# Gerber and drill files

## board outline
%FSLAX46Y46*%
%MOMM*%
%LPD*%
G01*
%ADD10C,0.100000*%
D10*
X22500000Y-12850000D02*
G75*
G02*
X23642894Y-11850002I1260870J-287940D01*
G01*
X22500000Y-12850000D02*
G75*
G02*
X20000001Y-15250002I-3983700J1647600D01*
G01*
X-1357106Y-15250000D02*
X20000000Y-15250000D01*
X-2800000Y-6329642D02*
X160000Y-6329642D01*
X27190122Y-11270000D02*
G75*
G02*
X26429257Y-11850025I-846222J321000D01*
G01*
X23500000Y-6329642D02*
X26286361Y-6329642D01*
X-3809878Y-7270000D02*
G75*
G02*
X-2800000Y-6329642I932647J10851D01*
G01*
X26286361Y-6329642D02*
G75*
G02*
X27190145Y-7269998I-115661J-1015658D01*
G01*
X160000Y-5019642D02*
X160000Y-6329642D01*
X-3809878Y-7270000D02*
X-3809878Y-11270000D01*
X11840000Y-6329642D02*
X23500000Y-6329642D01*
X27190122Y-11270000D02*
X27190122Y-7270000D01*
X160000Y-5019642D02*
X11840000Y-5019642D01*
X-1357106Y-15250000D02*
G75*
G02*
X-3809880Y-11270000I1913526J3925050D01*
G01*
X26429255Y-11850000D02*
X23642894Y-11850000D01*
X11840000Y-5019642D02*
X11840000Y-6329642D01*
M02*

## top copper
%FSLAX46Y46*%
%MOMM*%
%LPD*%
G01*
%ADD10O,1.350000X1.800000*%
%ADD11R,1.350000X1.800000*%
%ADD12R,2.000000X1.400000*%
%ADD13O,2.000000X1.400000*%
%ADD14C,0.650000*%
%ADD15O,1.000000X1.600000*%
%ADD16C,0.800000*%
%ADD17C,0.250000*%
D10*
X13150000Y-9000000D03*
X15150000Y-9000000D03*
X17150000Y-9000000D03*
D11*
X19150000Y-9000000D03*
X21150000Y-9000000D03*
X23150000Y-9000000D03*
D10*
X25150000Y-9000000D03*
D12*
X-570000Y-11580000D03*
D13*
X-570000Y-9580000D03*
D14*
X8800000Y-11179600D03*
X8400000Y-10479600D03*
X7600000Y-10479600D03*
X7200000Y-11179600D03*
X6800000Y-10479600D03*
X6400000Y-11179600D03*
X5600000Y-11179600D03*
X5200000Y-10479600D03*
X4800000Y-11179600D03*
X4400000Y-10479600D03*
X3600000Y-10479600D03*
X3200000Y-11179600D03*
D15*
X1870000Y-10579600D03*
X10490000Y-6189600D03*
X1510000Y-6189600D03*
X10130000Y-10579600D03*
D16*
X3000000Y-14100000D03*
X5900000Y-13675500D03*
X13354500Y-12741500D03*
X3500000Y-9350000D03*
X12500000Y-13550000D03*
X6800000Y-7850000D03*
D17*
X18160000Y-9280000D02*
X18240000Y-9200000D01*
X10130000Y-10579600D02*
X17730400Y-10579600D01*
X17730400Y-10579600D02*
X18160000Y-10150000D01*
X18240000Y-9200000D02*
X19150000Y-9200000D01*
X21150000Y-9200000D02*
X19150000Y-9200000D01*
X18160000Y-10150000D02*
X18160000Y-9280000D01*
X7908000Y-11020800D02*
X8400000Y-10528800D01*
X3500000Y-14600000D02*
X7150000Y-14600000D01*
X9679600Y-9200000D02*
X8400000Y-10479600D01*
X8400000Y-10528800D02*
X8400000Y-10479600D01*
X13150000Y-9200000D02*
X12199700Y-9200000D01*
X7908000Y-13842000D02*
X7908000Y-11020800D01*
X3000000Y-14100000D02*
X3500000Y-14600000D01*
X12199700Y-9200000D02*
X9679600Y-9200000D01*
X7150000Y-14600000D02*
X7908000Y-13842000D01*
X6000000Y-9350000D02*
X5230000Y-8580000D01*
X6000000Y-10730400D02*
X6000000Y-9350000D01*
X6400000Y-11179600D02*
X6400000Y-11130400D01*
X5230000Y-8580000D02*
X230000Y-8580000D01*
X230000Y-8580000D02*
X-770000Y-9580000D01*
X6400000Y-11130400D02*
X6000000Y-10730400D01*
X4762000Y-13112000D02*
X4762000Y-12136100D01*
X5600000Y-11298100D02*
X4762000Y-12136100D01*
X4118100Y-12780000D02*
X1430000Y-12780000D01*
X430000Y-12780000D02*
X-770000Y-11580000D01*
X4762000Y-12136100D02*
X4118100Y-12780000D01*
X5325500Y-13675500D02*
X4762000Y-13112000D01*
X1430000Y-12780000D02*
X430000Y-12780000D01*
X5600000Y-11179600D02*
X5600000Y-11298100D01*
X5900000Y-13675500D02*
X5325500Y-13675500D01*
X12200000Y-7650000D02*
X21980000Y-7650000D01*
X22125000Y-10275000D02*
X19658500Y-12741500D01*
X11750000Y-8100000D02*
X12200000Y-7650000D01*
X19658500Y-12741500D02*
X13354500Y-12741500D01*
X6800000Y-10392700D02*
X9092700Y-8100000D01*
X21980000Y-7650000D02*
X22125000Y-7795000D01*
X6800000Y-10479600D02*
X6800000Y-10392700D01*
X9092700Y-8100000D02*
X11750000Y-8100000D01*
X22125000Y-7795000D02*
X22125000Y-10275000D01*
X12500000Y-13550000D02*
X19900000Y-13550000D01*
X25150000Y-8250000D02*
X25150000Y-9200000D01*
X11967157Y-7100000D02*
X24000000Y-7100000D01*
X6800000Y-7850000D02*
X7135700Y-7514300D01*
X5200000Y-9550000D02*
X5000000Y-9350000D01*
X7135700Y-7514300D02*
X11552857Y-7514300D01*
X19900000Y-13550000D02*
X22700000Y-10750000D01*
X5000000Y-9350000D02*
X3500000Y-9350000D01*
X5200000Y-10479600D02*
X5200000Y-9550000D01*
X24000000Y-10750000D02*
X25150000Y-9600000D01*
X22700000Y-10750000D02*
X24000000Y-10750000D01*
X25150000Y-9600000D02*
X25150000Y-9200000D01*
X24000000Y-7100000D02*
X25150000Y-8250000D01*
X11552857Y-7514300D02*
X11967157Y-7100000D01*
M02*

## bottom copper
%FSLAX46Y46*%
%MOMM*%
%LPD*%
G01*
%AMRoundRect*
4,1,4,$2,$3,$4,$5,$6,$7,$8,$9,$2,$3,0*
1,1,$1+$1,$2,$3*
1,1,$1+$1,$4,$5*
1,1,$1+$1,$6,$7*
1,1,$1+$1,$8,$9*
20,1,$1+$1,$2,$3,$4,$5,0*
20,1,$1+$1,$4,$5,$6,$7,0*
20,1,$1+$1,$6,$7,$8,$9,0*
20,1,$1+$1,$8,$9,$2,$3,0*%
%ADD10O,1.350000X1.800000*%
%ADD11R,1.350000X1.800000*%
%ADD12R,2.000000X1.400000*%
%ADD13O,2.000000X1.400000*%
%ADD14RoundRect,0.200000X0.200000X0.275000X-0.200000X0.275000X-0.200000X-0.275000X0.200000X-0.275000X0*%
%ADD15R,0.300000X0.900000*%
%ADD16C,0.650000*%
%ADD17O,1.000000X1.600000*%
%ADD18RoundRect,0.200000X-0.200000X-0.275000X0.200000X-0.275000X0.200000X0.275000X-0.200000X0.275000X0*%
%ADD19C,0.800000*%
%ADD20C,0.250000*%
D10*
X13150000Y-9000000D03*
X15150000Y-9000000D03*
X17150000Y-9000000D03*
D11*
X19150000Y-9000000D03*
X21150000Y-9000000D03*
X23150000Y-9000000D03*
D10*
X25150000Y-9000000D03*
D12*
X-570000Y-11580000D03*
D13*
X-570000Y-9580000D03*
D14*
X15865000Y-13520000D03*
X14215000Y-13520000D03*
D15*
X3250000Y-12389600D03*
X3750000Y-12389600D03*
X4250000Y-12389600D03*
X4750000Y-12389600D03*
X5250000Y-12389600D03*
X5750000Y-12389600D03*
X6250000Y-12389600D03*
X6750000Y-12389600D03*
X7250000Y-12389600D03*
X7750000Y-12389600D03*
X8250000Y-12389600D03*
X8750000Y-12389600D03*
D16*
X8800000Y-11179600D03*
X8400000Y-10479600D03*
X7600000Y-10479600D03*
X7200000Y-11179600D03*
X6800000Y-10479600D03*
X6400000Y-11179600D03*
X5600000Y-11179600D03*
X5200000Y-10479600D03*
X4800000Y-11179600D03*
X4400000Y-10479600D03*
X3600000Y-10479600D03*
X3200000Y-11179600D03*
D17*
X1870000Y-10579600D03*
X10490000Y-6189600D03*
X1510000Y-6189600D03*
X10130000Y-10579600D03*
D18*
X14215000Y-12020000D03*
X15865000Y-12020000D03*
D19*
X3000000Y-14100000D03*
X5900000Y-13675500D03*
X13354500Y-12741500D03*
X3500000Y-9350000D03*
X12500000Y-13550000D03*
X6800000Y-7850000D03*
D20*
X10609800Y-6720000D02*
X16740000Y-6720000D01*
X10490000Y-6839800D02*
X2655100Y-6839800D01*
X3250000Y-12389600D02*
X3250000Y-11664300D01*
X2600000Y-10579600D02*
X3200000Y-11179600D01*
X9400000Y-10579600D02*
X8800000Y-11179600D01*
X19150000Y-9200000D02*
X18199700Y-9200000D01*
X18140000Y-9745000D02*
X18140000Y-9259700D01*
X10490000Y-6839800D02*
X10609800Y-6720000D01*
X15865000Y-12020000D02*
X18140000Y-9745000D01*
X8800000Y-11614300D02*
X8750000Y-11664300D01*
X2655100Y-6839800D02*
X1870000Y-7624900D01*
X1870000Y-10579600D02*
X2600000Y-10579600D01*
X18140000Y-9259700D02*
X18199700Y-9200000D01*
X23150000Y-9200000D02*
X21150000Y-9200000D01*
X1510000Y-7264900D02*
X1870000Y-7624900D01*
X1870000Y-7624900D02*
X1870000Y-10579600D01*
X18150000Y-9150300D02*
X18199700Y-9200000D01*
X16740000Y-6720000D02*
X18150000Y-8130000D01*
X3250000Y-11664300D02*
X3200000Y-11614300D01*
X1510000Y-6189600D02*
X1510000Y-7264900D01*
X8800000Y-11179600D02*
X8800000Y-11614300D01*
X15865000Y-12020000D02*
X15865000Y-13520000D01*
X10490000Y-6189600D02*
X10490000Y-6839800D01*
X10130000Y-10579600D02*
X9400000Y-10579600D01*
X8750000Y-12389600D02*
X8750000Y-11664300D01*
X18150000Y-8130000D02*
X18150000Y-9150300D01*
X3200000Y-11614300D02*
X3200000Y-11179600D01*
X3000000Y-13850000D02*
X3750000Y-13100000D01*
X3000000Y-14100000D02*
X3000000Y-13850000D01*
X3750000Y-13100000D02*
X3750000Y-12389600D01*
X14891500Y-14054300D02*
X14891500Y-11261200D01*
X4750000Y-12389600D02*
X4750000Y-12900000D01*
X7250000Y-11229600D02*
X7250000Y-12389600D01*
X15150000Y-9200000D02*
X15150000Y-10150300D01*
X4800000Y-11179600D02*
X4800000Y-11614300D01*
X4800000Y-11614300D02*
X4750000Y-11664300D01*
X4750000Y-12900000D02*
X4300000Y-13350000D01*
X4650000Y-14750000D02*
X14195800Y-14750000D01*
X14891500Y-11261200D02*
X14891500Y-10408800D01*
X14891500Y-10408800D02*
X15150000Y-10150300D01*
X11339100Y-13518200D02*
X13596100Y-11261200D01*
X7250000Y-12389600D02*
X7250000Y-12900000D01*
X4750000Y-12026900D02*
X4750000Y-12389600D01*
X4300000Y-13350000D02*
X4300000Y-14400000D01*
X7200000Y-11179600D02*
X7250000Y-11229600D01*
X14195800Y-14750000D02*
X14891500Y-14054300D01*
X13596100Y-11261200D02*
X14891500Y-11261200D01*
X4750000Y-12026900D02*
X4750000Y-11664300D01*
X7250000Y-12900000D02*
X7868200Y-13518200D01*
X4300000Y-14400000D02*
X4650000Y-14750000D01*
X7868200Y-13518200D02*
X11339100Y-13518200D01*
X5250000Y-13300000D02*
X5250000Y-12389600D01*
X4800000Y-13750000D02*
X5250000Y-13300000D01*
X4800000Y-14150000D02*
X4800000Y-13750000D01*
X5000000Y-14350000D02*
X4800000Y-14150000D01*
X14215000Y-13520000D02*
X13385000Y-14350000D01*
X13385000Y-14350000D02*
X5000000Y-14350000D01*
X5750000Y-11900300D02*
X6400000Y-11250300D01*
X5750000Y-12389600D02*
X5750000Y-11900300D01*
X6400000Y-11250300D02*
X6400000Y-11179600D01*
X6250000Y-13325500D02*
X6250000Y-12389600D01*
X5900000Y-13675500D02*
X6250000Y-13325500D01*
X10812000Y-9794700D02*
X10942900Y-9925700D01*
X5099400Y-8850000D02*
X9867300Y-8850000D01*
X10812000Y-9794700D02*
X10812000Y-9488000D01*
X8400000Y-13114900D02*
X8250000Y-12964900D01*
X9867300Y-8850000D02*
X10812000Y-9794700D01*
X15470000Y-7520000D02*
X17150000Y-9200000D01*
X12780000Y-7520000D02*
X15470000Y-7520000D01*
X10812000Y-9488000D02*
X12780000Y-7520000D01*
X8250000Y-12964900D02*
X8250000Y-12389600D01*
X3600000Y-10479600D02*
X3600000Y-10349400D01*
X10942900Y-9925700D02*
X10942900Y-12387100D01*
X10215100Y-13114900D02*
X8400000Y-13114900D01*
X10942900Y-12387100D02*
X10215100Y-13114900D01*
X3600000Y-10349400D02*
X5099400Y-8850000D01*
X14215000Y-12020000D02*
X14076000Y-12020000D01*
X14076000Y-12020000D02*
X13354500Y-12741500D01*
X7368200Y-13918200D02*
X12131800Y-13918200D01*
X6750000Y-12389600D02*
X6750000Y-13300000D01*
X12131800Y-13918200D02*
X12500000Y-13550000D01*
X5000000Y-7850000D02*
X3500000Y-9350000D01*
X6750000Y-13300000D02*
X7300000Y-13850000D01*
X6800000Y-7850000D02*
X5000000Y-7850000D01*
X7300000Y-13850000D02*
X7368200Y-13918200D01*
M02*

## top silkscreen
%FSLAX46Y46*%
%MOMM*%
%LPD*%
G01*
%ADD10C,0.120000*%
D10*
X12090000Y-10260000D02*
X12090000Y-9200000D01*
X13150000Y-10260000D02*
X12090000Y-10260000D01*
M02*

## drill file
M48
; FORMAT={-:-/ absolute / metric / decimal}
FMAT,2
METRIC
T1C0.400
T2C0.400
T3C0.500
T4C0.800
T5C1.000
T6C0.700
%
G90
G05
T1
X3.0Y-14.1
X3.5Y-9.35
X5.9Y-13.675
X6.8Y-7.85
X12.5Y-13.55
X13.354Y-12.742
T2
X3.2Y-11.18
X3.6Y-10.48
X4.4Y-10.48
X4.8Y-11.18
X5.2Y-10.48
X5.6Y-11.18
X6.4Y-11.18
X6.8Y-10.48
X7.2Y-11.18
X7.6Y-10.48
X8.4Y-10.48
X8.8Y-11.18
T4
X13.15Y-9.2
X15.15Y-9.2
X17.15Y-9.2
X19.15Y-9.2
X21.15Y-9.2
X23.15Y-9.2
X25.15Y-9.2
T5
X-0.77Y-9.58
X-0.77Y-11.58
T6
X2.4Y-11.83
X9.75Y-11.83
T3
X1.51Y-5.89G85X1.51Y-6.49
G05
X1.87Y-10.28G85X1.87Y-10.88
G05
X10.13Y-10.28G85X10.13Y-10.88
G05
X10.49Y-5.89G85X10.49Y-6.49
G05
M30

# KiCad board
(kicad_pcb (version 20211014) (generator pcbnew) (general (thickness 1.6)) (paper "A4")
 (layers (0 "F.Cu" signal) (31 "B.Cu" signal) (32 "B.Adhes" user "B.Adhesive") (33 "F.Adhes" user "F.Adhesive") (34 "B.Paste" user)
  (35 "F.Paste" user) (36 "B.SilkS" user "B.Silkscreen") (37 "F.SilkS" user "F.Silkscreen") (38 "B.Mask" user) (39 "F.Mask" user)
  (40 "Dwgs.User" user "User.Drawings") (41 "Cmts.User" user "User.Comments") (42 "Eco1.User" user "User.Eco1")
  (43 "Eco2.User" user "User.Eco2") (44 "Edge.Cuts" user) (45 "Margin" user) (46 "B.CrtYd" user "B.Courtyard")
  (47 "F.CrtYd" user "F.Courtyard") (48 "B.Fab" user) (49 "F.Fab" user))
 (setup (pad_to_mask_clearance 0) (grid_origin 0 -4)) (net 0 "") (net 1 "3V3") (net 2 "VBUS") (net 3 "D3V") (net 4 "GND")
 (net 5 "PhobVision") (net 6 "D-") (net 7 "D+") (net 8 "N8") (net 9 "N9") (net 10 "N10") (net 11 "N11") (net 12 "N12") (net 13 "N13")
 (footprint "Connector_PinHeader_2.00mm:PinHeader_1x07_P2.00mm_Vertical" (layer "F.Cu") (at 13.15 9.2 90)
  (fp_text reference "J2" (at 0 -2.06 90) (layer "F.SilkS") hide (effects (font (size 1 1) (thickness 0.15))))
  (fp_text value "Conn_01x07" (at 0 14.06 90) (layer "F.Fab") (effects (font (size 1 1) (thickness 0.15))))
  (fp_line (start -1.06 -1.06) (end 0 -1.06) (layer "F.SilkS") (width 0.12))
  (fp_line (start -1.06 0) (end -1.06 -1.06) (layer "F.SilkS") (width 0.12))
  (pad "1" thru_hole oval (at 0 0 90) (size 1.8 1.35) (drill 0.8 (offset 0.2 0)) (layers F&B.Cu *.Mask) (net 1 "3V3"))
  (pad "2" thru_hole oval (at 0 2 90) (size 1.8 1.35) (drill 0.8 (offset 0.2 0)) (layers F&B.Cu *.Mask) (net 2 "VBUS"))
  (pad "3" thru_hole oval (at 0 4 90) (size 1.8 1.35) (drill 0.8 (offset 0.2 0)) (layers F&B.Cu *.Mask) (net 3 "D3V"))
  (pad "4" thru_hole rect (at 0 6 90) (size 1.8 1.35) (drill 0.8 (offset 0.2 0)) (layers F&B.Cu *.Mask) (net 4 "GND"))
  (pad "5" thru_hole rect (at 0 8 90) (size 1.8 1.35) (drill 0.8 (offset 0.2 0)) (layers F&B.Cu *.Mask) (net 4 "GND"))
  (pad "6" thru_hole rect (at 0 10 90) (size 1.8 1.35) (drill 0.8 (offset 0.2 0)) (layers F&B.Cu *.Mask) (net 4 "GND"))
  (pad "7" thru_hole oval (at 0 12 90) (size 1.8 1.35) (drill 0.8 (offset 0.2 0)) (layers F&B.Cu *.Mask) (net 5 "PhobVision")))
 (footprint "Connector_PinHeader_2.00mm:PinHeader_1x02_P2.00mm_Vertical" (layer "B.Cu") (at -0.77 11.58)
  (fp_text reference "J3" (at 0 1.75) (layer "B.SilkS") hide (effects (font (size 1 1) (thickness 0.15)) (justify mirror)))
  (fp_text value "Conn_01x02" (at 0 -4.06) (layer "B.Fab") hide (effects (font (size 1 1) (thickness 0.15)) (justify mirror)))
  (pad "1" thru_hole rect locked (at 0 0) (size 2 1.4) (drill 1 (offset 0.2 0)) (layers F&B.Cu *.Mask) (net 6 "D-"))
  (pad "2" thru_hole oval locked (at 0 -2) (size 2 1.4) (drill 1 (offset 0.2 0)) (layers F&B.Cu *.Mask) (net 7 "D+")))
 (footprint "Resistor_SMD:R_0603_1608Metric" (layer "B.Cu") (at 15.04 13.52 180)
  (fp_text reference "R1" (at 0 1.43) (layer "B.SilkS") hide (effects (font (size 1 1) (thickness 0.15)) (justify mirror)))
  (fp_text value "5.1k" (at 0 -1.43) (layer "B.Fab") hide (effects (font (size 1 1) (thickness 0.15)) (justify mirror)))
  (pad "1" smd roundrect locked (at -0.825 0 180) (size 0.8 0.95) (layers "B.Cu" "B.Paste" "B.Mask") (roundrect_rratio 0.25) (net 4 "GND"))
  (pad "2" smd roundrect locked (at 0.825 0 180) (size 0.8 0.95) (layers "B.Cu" "B.Paste" "B.Mask") (roundrect_rratio 0.25) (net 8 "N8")))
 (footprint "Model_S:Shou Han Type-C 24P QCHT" (layer "B.Cu") (at 6 4.3296)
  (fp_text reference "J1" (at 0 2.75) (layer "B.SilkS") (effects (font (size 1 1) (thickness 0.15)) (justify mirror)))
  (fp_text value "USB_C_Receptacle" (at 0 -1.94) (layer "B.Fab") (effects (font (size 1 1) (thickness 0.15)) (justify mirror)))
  (pad "" np_thru_hole circle (at -3.6 7.5) (size 0.7 0.7) (drill 0.7) (layers F&B.Cu *.Mask))
  (pad "" np_thru_hole circle (at 3.75 7.5) (size 0.7 0.7) (drill 0.7) (layers F&B.Cu *.Mask))
  (pad "A1" smd rect (at -2.75 8.06) (size 0.3 0.9) (layers "B.Cu" "B.Paste" "B.Mask") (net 4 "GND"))
  (pad "A2" smd rect (at -2.25 8.06) (size 0.3 0.9) (layers "B.Cu" "B.Paste" "B.Mask") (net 1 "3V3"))
  (pad "A3" smd rect (at -1.75 8.06) (size 0.3 0.9) (layers "B.Cu" "B.Paste" "B.Mask") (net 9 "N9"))
  (pad "A4" smd rect (at -1.25 8.06) (size 0.3 0.9) (layers "B.Cu" "B.Paste" "B.Mask") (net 2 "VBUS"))
  (pad "A5" smd rect (at -0.75 8.06) (size 0.3 0.9) (layers "B.Cu" "B.Paste" "B.Mask") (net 8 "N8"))
  (pad "A6" smd rect (at -0.25 8.06) (size 0.3 0.9) (layers "B.Cu" "B.Paste" "B.Mask") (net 7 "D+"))
  (pad "A7" smd rect (at 0.25 8.06) (size 0.3 0.9) (layers "B.Cu" "B.Paste" "B.Mask") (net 6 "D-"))
  (pad "A8" smd rect (at 0.75 8.06) (size 0.3 0.9) (layers "B.Cu" "B.Paste" "B.Mask") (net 5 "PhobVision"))
  (pad "A9" smd rect (at 1.25 8.06) (size 0.3 0.9) (layers "B.Cu" "B.Paste" "B.Mask") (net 2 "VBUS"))
  (pad "A10" smd rect (at 1.75 8.06) (size 0.3 0.9) (layers "B.Cu" "B.Paste" "B.Mask") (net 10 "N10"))
  (pad "A11" smd rect (at 2.25 8.06) (size 0.3 0.9) (layers "B.Cu" "B.Paste" "B.Mask") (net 3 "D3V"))
  (pad "A12" smd rect (at 2.75 8.06) (size 0.3 0.9) (layers "B.Cu" "B.Paste" "B.Mask") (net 4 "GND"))
  (pad "B1" thru_hole circle (at 2.8 6.85) (size 0.65 0.65) (drill 0.4) (layers F&B.Cu *.Mask) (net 4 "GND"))
  (pad "B2" thru_hole circle (at 2.4 6.15) (size 0.65 0.65) (drill 0.4) (layers F&B.Cu *.Mask) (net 1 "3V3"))
  (pad "B3" thru_hole circle (at 1.6 6.15) (size 0.65 0.65) (drill 0.4) (layers F&B.Cu *.Mask) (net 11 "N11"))
  (pad "B4" thru_hole circle (at 1.2 6.85) (size 0.65 0.65) (drill 0.4) (layers F&B.Cu *.Mask) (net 2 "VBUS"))
  (pad "B5" thru_hole circle (at 0.8 6.15) (size 0.65 0.65) (drill 0.4) (layers F&B.Cu *.Mask) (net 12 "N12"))
  (pad "B6" thru_hole circle (at 0.4 6.85) (size 0.65 0.65) (drill 0.4) (layers F&B.Cu *.Mask) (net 7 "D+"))
  (pad "B7" thru_hole circle (at -0.4 6.85) (size 0.65 0.65) (drill 0.4) (layers F&B.Cu *.Mask) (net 6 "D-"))
  (pad "B8" thru_hole circle (at -0.8 6.15) (size 0.65 0.65) (drill 0.4) (layers F&B.Cu *.Mask) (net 5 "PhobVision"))
  (pad "B9" thru_hole circle (at -1.2 6.85) (size 0.65 0.65) (drill 0.4) (layers F&B.Cu *.Mask) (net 2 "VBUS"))
  (pad "B10" thru_hole circle (at -1.6 6.15) (size 0.65 0.65) (drill 0.4) (layers F&B.Cu *.Mask) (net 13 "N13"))
  (pad "B11" thru_hole circle (at -2.4 6.15) (size 0.65 0.65) (drill 0.4) (layers F&B.Cu *.Mask) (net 3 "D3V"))
  (pad "B12" thru_hole circle (at -2.8 6.85) (size 0.65 0.65) (drill 0.4) (layers F&B.Cu *.Mask) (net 4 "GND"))
  (pad "S1" thru_hole oval (at -4.13 6.25) (size 1 1.6) (drill oval 0.5 1.1) (layers F&B.Cu *.Mask) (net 4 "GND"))
  (pad "S1" thru_hole oval (at 4.49 1.86) (size 1 1.6) (drill oval 0.5 1.1) (layers F&B.Cu *.Mask) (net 4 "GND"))
  (pad "S1" thru_hole oval (at -4.49 1.86) (size 1 1.6) (drill oval 0.5 1.1) (layers F&B.Cu *.Mask) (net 4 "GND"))
  (pad "S1" thru_hole oval (at 4.13 6.25) (size 1 1.6) (drill oval 0.5 1.1) (layers F&B.Cu *.Mask) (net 4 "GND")))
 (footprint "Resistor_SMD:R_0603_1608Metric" (layer "B.Cu") (at 15.04 12.02)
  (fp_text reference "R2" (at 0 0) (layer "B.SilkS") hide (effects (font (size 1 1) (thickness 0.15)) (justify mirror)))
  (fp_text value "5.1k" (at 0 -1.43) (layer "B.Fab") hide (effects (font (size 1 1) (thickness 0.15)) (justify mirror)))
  (pad "1" smd roundrect locked (at -0.825 0) (size 0.8 0.95) (layers "B.Cu" "B.Paste" "B.Mask") (roundrect_rratio 0.25) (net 12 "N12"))
  (pad "2" smd roundrect locked (at 0.825 0) (size 0.8 0.95) (layers "B.Cu" "B.Paste" "B.Mask") (roundrect_rratio 0.25) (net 4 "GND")))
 (gr_arc (start 22.5 12.85) (mid 22.909223 12.164595) (end 23.642894 11.85) (layer "Edge.Cuts") (width 0.1))
 (gr_arc (start 22.5 12.85) (mid 21.501783 14.312274) (end 20 15.25) (layer "Edge.Cuts") (width 0.1))
 (gr_line (start -1.357106 15.25) (end 20 15.25) (layer "Edge.Cuts") (width 0.1))
 (gr_line (start -2.8 6.329642) (end 0.16 6.329642) (layer "Edge.Cuts") (width 0.1))
 (gr_arc (start 27.190122 11.27) (mid 26.892588 11.668751) (end 26.429255 11.85) (layer "Edge.Cuts") (width 0.1))
 (gr_line (start 23.5 6.329642) (end 26.286361 6.329642) (layer "Edge.Cuts") (width 0.1))
 (gr_arc (start -3.809878 7.27) (mid -3.512843 6.576547) (end -2.8 6.329642) (layer "Edge.Cuts") (width 0.1))
 (gr_arc (start 26.286361 6.329642) (mid 26.907696 6.636961) (end 27.190122 7.27) (layer "Edge.Cuts") (width 0.1))
 (gr_line (start 0.16 5.019642) (end 0.16 6.329642) (layer "Edge.Cuts") (width 0.1))
 (gr_line (start -3.809878 7.27) (end -3.809878 11.27) (layer "Edge.Cuts") (width 0.1))
 (gr_line (start 11.84 6.329642) (end 23.5 6.329642) (layer "Edge.Cuts") (width 0.1))
 (gr_line (start 27.190122 11.27) (end 27.190122 7.27) (layer "Edge.Cuts") (width 0.1))
 (gr_line (start 0.16 5.019642) (end 11.84 5.019642) (layer "Edge.Cuts") (width 0.1))
 (gr_arc (start -1.357106 15.25) (mid -3.160991 13.615898) (end -3.809878 11.27) (layer "Edge.Cuts") (width 0.1))
 (gr_line (start 26.429255 11.85) (end 23.642894 11.85) (layer "Edge.Cuts") (width 0.1))
 (gr_line (start 11.84 5.019642) (end 11.84 6.329642) (layer "Edge.Cuts") (width 0.1))
 (segment (start 18.16 9.28) (end 18.24 9.2) (width 0.25) (layer "F.Cu") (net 4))
 (segment (start 10.13 10.5796) (end 17.7304 10.5796) (width 0.25) (layer "F.Cu") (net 4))
 (segment (start 17.7304 10.5796) (end 18.16 10.15) (width 0.25) (layer "F.Cu") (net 4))
 (segment (start 18.24 9.2) (end 19.15 9.2) (width 0.25) (layer "F.Cu") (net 4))
 (segment (start 21.15 9.2) (end 19.15 9.2) (width 0.25) (layer "F.Cu") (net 4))
 (segment (start 18.16 10.15) (end 18.16 9.28) (width 0.25) (layer "F.Cu") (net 4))
 (segment (start 10.6098 6.72) (end 16.74 6.72) (width 0.25) (layer "B.Cu") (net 4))
 (segment (start 10.49 6.8398) (end 2.6551 6.8398) (width 0.25) (layer "B.Cu") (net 4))
 (segment (start 3.25 12.3896) (end 3.25 11.6643) (width 0.25) (layer "B.Cu") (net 4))
 (segment (start 2.6 10.5796) (end 3.2 11.1796) (width 0.25) (layer "B.Cu") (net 4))
 (segment (start 9.4 10.5796) (end 8.8 11.1796) (width 0.25) (layer "B.Cu") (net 4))
 (segment (start 19.15 9.2) (end 18.1997 9.2) (width 0.25) (layer "B.Cu") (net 4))
 (segment (start 18.14 9.745) (end 18.14 9.2597) (width 0.25) (layer "B.Cu") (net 4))
 (segment (start 10.49 6.8398) (end 10.6098 6.72) (width 0.25) (layer "B.Cu") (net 4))
 (segment (start 15.865 12.02) (end 18.14 9.745) (width 0.25) (layer "B.Cu") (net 4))
 (segment (start 8.8 11.6143) (end 8.75 11.6643) (width 0.25) (layer "B.Cu") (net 4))
 (segment (start 2.6551 6.8398) (end 1.87 7.6249) (width 0.25) (layer "B.Cu") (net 4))
 (segment (start 1.87 10.5796) (end 2.6 10.5796) (width 0.25) (layer "B.Cu") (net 4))
 (segment (start 18.14 9.2597) (end 18.1997 9.2) (width 0.25) (layer "B.Cu") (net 4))
 (segment (start 23.15 9.2) (end 21.15 9.2) (width 0.25) (layer "B.Cu") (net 4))
 (segment (start 1.51 7.2649) (end 1.87 7.6249) (width 0.25) (layer "B.Cu") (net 4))
 (segment (start 1.87 7.6249) (end 1.87 10.5796) (width 0.25) (layer "B.Cu") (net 4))
 (segment (start 18.15 9.1503) (end 18.1997 9.2) (width 0.25) (layer "B.Cu") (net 4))
 (segment (start 16.74 6.72) (end 18.15 8.13) (width 0.25) (layer "B.Cu") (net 4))
 (segment (start 3.25 11.6643) (end 3.2 11.6143) (width 0.25) (layer "B.Cu") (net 4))
 (segment (start 1.51 6.1896) (end 1.51 7.2649) (width 0.25) (layer "B.Cu") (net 4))
 (segment (start 8.8 11.1796) (end 8.8 11.6143) (width 0.25) (layer "B.Cu") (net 4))
 (segment (start 15.865 12.02) (end 15.865 13.52) (width 0.25) (layer "B.Cu") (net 4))
 (segment (start 10.49 6.1896) (end 10.49 6.8398) (width 0.25) (layer "B.Cu") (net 4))
 (segment (start 10.13 10.5796) (end 9.4 10.5796) (width 0.25) (layer "B.Cu") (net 4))
 (segment (start 8.75 12.3896) (end 8.75 11.6643) (width 0.25) (layer "B.Cu") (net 4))
 (segment (start 18.15 8.13) (end 18.15 9.1503) (width 0.25) (layer "B.Cu") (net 4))
 (segment (start 3.2 11.6143) (end 3.2 11.1796) (width 0.25) (layer "B.Cu") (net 4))
 (segment (start 7.908 11.0208) (end 8.4 10.5288) (width 0.25) (layer "F.Cu") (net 1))
 (segment (start 3.5 14.6) (end 7.15 14.6) (width 0.25) (layer "F.Cu") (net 1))
 (segment (start 9.6796 9.2) (end 8.4 10.4796) (width 0.25) (layer "F.Cu") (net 1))
 (segment (start 8.4 10.5288) (end 8.4 10.4796) (width 0.25) (layer "F.Cu") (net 1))
 (segment (start 13.15 9.2) (end 12.1997 9.2) (width 0.25) (layer "F.Cu") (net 1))
 (segment (start 7.908 13.842) (end 7.908 11.0208) (width 0.25) (layer "F.Cu") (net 1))
 (segment (start 3 14.1) (end 3.5 14.6) (width 0.25) (layer "F.Cu") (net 1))
 (segment (start 12.1997 9.2) (end 9.6796 9.2) (width 0.25) (layer "F.Cu") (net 1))
 (segment (start 7.15 14.6) (end 7.908 13.842) (width 0.25) (layer "F.Cu") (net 1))
 (via (at 3 14.1) (size 0.8) (drill 0.4) (layers "F.Cu" "B.Cu") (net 1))
 (segment (start 3 13.85) (end 3.75 13.1) (width 0.25) (layer "B.Cu") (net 1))
 (segment (start 3 14.1) (end 3 13.85) (width 0.25) (layer "B.Cu") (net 1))
 (segment (start 3.75 13.1) (end 3.75 12.3896) (width 0.25) (layer "B.Cu") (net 1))
 (segment (start 14.8915 14.0543) (end 14.8915 11.2612) (width 0.25) (layer "B.Cu") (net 2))
 (segment (start 4.75 12.3896) (end 4.75 12.9) (width 0.25) (layer "B.Cu") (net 2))
 (segment (start 7.25 11.2296) (end 7.25 12.3896) (width 0.25) (layer "B.Cu") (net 2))
 (segment (start 15.15 9.2) (end 15.15 10.1503) (width 0.25) (layer "B.Cu") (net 2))
 (segment (start 4.8 11.1796) (end 4.8 11.6143) (width 0.25) (layer "B.Cu") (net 2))
 (segment (start 4.8 11.6143) (end 4.75 11.6643) (width 0.25) (layer "B.Cu") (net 2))
 (segment (start 4.75 12.9) (end 4.3 13.35) (width 0.25) (layer "B.Cu") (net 2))
 (segment (start 4.65 14.75) (end 14.1958 14.75) (width 0.25) (layer "B.Cu") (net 2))
 (segment (start 14.8915 11.2612) (end 14.8915 10.4088) (width 0.25) (layer "B.Cu") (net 2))
 (segment (start 14.8915 10.4088) (end 15.15 10.1503) (width 0.25) (layer "B.Cu") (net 2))
 (segment (start 11.3391 13.5182) (end 13.5961 11.2612) (width 0.25) (layer "B.Cu") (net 2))
 (segment (start 7.25 12.3896) (end 7.25 12.9) (width 0.25) (layer "B.Cu") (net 2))
 (segment (start 4.75 12.0269) (end 4.75 12.3896) (width 0.25) (layer "B.Cu") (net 2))
 (segment (start 4.3 13.35) (end 4.3 14.4) (width 0.25) (layer "B.Cu") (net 2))
 (segment (start 7.2 11.1796) (end 7.25 11.2296) (width 0.25) (layer "B.Cu") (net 2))
 (segment (start 14.1958 14.75) (end 14.8915 14.0543) (width 0.25) (layer "B.Cu") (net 2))
 (segment (start 13.5961 11.2612) (end 14.8915 11.2612) (width 0.25) (layer "B.Cu") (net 2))
 (segment (start 4.75 12.0269) (end 4.75 11.6643) (width 0.25) (layer "B.Cu") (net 2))
 (segment (start 7.25 12.9) (end 7.8682 13.5182) (width 0.25) (layer "B.Cu") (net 2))
 (segment (start 4.3 14.4) (end 4.65 14.75) (width 0.25) (layer "B.Cu") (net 2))
 (segment (start 7.8682 13.5182) (end 11.3391 13.5182) (width 0.25) (layer "B.Cu") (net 2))
 (segment (start 5.25 13.3) (end 5.25 12.3896) (width 0.25) (layer "B.Cu") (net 8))
 (segment (start 4.8 13.75) (end 5.25 13.3) (width 0.25) (layer "B.Cu") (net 8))
 (segment (start 4.8 14.15) (end 4.8 13.75) (width 0.25) (layer "B.Cu") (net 8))
 (segment (start 5 14.35) (end 4.8 14.15) (width 0.25) (layer "B.Cu") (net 8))
 (segment (start 14.215 13.52) (end 13.385 14.35) (width 0.25) (layer "B.Cu") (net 8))
 (segment (start 13.385 14.35) (end 5 14.35) (width 0.25) (layer "B.Cu") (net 8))
 (segment (start 6 9.35) (end 5.23 8.58) (width 0.25) (layer "F.Cu") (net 7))
 (segment (start 6 10.7304) (end 6 9.35) (width 0.25) (layer "F.Cu") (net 7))
 (segment (start 6.4 11.1796) (end 6.4 11.1304) (width 0.25) (layer "F.Cu") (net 7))
 (segment (start 5.23 8.58) (end 0.23 8.58) (width 0.25) (layer "F.Cu") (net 7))
 (segment (start 0.23 8.58) (end -0.77 9.58) (width 0.25) (layer "F.Cu") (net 7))
 (segment (start 6.4 11.1304) (end 6 10.7304) (width 0.25) (layer "F.Cu") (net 7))
 (segment (start 5.75 11.9003) (end 6.4 11.2503) (width 0.25) (layer "B.Cu") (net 7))
 (segment (start 5.75 12.3896) (end 5.75 11.9003) (width 0.25) (layer "B.Cu") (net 7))
 (segment (start 6.4 11.2503) (end 6.4 11.1796) (width 0.25) (layer "B.Cu") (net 7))
 (segment (start 4.762 13.112) (end 4.762 12.1361) (width 0.25) (layer "F.Cu") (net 6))
 (segment (start 5.6 11.2981) (end 4.762 12.1361) (width 0.25) (layer "F.Cu") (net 6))
 (segment (start 4.1181 12.78) (end 1.43 12.78) (width 0.25) (layer "F.Cu") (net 6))
 (segment (start 0.43 12.78) (end -0.77 11.58) (width 0.25) (layer "F.Cu") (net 6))
 (segment (start 4.762 12.1361) (end 4.1181 12.78) (width 0.25) (layer "F.Cu") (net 6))
 (segment (start 5.3255 13.6755) (end 4.762 13.112) (width 0.25) (layer "F.Cu") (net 6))
 (segment (start 1.43 12.78) (end 0.43 12.78) (width 0.25) (layer "F.Cu") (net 6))
 (segment (start 5.6 11.1796) (end 5.6 11.2981) (width 0.25) (layer "F.Cu") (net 6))
 (segment (start 5.9 13.6755) (end 5.3255 13.6755) (width 0.25) (layer "F.Cu") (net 6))
 (via (at 5.9 13.6755) (size 0.8) (drill 0.4) (layers "F.Cu" "B.Cu") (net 6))
 (segment (start 6.25 13.3255) (end 6.25 12.3896) (width 0.25) (layer "B.Cu") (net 6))
 (segment (start 5.9 13.6755) (end 6.25 13.3255) (width 0.25) (layer "B.Cu") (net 6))
 (segment (start 10.812 9.7947) (end 10.9429 9.9257) (width 0.25) (layer "B.Cu") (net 3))
 (segment (start 5.0994 8.85) (end 9.8673 8.85) (width 0.25) (layer "B.Cu") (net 3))
 (segment (start 10.812 9.7947) (end 10.812 9.488) (width 0.25) (layer "B.Cu") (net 3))
 (segment (start 8.4 13.1149) (end 8.25 12.9649) (width 0.25) (layer "B.Cu") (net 3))
 (segment (start 9.8673 8.85) (end 10.812 9.7947) (width 0.25) (layer "B.Cu") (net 3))
 (segment (start 15.47 7.52) (end 17.15 9.2) (width 0.25) (layer "B.Cu") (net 3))
 (segment (start 12.78 7.52) (end 15.47 7.52) (width 0.25) (layer "B.Cu") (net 3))
 (segment (start 10.812 9.488) (end 12.78 7.52) (width 0.25) (layer "B.Cu") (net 3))
 (segment (start 8.25 12.9649) (end 8.25 12.3896) (width 0.25) (layer "B.Cu") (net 3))
 (segment (start 3.6 10.4796) (end 3.6 10.3494) (width 0.25) (layer "B.Cu") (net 3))
 (segment (start 10.9429 9.9257) (end 10.9429 12.3871) (width 0.25) (layer "B.Cu") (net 3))
 (segment (start 10.2151 13.1149) (end 8.4 13.1149) (width 0.25) (layer "B.Cu") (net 3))
 (segment (start 10.9429 12.3871) (end 10.2151 13.1149) (width 0.25) (layer "B.Cu") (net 3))
 (segment (start 3.6 10.3494) (end 5.0994 8.85) (width 0.25) (layer "B.Cu") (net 3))
 (segment (start 12.2 7.65) (end 21.98 7.65) (width 0.25) (layer "F.Cu") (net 12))
 (segment (start 22.125 10.275) (end 19.6585 12.7415) (width 0.25) (layer "F.Cu") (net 12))
 (segment (start 11.75 8.1) (end 12.2 7.65) (width 0.25) (layer "F.Cu") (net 12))
 (segment (start 19.6585 12.7415) (end 13.3545 12.7415) (width 0.25) (layer "F.Cu") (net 12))
 (segment (start 6.8 10.3927) (end 9.0927 8.1) (width 0.25) (layer "F.Cu") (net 12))
 (segment (start 21.98 7.65) (end 22.125 7.795) (width 0.25) (layer "F.Cu") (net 12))
 (segment (start 6.8 10.4796) (end 6.8 10.3927) (width 0.25) (layer "F.Cu") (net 12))
 (segment (start 9.0927 8.1) (end 11.75 8.1) (width 0.25) (layer "F.Cu") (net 12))
 (segment (start 22.125 7.795) (end 22.125 10.275) (width 0.25) (layer "F.Cu") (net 12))
 (via (at 13.3545 12.7415) (size 0.8) (drill 0.4) (layers "F.Cu" "B.Cu") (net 12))
 (segment (start 14.215 12.02) (end 14.076 12.02) (width 0.25) (layer "B.Cu") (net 12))
 (segment (start 14.076 12.02) (end 13.3545 12.7415) (width 0.25) (layer "B.Cu") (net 12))
 (segment (start 12.5 13.55) (end 19.9 13.55) (width 0.25) (layer "F.Cu") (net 5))
 (segment (start 25.15 8.25) (end 25.15 9.2) (width 0.25) (layer "F.Cu") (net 5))
 (segment (start 11.967157 7.1) (end 24 7.1) (width 0.25) (layer "F.Cu") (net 5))
 (segment (start 6.8 7.85) (end 7.1357 7.5143) (width 0.25) (layer "F.Cu") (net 5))
 (segment (start 5.2 9.55) (end 5 9.35) (width 0.25) (layer "F.Cu") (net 5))
 (segment (start 7.1357 7.5143) (end 11.552857 7.5143) (width 0.25) (layer "F.Cu") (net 5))
 (segment (start 19.9 13.55) (end 22.7 10.75) (width 0.25) (layer "F.Cu") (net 5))
 (segment (start 5 9.35) (end 3.5 9.35) (width 0.25) (layer "F.Cu") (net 5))
 (segment (start 5.2 10.4796) (end 5.2 9.55) (width 0.25) (layer "F.Cu") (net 5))
 (segment (start 24 10.75) (end 25.15 9.6) (width 0.25) (layer "F.Cu") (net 5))
 (segment (start 22.7 10.75) (end 24 10.75) (width 0.25) (layer "F.Cu") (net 5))
 (segment (start 25.15 9.6) (end 25.15 9.2) (width 0.25) (layer "F.Cu") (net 5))
 (segment (start 24 7.1) (end 25.15 8.25) (width 0.25) (layer "F.Cu") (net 5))
 (segment (start 11.552857 7.5143) (end 11.967157 7.1) (width 0.25) (layer "F.Cu") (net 5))
 (via (at 3.5 9.35) (size 0.8) (drill 0.4) (layers "F.Cu" "B.Cu") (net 5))
 (via (at 12.5 13.55) (size 0.8) (drill 0.4) (layers "F.Cu" "B.Cu") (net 5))
 (via (at 6.8 7.85) (size 0.8) (drill 0.4) (layers "F.Cu" "B.Cu") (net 5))
 (segment (start 7.3682 13.9182) (end 12.1318 13.9182) (width 0.25) (layer "B.Cu") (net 5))
 (segment (start 6.75 12.3896) (end 6.75 13.3) (width 0.25) (layer "B.Cu") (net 5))
 (segment (start 12.1318 13.9182) (end 12.5 13.55) (width 0.25) (layer "B.Cu") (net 5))
 (segment (start 5 7.85) (end 3.5 9.35) (width 0.25) (layer "B.Cu") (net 5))
 (segment (start 6.75 13.3) (end 7.3 13.85) (width 0.25) (layer "B.Cu") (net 5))
 (segment (start 6.8 7.85) (end 5 7.85) (width 0.25) (layer "B.Cu") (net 5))
 (segment (start 7.3 13.85) (end 7.3682 13.9182) (width 0.25) (layer "B.Cu") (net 5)))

